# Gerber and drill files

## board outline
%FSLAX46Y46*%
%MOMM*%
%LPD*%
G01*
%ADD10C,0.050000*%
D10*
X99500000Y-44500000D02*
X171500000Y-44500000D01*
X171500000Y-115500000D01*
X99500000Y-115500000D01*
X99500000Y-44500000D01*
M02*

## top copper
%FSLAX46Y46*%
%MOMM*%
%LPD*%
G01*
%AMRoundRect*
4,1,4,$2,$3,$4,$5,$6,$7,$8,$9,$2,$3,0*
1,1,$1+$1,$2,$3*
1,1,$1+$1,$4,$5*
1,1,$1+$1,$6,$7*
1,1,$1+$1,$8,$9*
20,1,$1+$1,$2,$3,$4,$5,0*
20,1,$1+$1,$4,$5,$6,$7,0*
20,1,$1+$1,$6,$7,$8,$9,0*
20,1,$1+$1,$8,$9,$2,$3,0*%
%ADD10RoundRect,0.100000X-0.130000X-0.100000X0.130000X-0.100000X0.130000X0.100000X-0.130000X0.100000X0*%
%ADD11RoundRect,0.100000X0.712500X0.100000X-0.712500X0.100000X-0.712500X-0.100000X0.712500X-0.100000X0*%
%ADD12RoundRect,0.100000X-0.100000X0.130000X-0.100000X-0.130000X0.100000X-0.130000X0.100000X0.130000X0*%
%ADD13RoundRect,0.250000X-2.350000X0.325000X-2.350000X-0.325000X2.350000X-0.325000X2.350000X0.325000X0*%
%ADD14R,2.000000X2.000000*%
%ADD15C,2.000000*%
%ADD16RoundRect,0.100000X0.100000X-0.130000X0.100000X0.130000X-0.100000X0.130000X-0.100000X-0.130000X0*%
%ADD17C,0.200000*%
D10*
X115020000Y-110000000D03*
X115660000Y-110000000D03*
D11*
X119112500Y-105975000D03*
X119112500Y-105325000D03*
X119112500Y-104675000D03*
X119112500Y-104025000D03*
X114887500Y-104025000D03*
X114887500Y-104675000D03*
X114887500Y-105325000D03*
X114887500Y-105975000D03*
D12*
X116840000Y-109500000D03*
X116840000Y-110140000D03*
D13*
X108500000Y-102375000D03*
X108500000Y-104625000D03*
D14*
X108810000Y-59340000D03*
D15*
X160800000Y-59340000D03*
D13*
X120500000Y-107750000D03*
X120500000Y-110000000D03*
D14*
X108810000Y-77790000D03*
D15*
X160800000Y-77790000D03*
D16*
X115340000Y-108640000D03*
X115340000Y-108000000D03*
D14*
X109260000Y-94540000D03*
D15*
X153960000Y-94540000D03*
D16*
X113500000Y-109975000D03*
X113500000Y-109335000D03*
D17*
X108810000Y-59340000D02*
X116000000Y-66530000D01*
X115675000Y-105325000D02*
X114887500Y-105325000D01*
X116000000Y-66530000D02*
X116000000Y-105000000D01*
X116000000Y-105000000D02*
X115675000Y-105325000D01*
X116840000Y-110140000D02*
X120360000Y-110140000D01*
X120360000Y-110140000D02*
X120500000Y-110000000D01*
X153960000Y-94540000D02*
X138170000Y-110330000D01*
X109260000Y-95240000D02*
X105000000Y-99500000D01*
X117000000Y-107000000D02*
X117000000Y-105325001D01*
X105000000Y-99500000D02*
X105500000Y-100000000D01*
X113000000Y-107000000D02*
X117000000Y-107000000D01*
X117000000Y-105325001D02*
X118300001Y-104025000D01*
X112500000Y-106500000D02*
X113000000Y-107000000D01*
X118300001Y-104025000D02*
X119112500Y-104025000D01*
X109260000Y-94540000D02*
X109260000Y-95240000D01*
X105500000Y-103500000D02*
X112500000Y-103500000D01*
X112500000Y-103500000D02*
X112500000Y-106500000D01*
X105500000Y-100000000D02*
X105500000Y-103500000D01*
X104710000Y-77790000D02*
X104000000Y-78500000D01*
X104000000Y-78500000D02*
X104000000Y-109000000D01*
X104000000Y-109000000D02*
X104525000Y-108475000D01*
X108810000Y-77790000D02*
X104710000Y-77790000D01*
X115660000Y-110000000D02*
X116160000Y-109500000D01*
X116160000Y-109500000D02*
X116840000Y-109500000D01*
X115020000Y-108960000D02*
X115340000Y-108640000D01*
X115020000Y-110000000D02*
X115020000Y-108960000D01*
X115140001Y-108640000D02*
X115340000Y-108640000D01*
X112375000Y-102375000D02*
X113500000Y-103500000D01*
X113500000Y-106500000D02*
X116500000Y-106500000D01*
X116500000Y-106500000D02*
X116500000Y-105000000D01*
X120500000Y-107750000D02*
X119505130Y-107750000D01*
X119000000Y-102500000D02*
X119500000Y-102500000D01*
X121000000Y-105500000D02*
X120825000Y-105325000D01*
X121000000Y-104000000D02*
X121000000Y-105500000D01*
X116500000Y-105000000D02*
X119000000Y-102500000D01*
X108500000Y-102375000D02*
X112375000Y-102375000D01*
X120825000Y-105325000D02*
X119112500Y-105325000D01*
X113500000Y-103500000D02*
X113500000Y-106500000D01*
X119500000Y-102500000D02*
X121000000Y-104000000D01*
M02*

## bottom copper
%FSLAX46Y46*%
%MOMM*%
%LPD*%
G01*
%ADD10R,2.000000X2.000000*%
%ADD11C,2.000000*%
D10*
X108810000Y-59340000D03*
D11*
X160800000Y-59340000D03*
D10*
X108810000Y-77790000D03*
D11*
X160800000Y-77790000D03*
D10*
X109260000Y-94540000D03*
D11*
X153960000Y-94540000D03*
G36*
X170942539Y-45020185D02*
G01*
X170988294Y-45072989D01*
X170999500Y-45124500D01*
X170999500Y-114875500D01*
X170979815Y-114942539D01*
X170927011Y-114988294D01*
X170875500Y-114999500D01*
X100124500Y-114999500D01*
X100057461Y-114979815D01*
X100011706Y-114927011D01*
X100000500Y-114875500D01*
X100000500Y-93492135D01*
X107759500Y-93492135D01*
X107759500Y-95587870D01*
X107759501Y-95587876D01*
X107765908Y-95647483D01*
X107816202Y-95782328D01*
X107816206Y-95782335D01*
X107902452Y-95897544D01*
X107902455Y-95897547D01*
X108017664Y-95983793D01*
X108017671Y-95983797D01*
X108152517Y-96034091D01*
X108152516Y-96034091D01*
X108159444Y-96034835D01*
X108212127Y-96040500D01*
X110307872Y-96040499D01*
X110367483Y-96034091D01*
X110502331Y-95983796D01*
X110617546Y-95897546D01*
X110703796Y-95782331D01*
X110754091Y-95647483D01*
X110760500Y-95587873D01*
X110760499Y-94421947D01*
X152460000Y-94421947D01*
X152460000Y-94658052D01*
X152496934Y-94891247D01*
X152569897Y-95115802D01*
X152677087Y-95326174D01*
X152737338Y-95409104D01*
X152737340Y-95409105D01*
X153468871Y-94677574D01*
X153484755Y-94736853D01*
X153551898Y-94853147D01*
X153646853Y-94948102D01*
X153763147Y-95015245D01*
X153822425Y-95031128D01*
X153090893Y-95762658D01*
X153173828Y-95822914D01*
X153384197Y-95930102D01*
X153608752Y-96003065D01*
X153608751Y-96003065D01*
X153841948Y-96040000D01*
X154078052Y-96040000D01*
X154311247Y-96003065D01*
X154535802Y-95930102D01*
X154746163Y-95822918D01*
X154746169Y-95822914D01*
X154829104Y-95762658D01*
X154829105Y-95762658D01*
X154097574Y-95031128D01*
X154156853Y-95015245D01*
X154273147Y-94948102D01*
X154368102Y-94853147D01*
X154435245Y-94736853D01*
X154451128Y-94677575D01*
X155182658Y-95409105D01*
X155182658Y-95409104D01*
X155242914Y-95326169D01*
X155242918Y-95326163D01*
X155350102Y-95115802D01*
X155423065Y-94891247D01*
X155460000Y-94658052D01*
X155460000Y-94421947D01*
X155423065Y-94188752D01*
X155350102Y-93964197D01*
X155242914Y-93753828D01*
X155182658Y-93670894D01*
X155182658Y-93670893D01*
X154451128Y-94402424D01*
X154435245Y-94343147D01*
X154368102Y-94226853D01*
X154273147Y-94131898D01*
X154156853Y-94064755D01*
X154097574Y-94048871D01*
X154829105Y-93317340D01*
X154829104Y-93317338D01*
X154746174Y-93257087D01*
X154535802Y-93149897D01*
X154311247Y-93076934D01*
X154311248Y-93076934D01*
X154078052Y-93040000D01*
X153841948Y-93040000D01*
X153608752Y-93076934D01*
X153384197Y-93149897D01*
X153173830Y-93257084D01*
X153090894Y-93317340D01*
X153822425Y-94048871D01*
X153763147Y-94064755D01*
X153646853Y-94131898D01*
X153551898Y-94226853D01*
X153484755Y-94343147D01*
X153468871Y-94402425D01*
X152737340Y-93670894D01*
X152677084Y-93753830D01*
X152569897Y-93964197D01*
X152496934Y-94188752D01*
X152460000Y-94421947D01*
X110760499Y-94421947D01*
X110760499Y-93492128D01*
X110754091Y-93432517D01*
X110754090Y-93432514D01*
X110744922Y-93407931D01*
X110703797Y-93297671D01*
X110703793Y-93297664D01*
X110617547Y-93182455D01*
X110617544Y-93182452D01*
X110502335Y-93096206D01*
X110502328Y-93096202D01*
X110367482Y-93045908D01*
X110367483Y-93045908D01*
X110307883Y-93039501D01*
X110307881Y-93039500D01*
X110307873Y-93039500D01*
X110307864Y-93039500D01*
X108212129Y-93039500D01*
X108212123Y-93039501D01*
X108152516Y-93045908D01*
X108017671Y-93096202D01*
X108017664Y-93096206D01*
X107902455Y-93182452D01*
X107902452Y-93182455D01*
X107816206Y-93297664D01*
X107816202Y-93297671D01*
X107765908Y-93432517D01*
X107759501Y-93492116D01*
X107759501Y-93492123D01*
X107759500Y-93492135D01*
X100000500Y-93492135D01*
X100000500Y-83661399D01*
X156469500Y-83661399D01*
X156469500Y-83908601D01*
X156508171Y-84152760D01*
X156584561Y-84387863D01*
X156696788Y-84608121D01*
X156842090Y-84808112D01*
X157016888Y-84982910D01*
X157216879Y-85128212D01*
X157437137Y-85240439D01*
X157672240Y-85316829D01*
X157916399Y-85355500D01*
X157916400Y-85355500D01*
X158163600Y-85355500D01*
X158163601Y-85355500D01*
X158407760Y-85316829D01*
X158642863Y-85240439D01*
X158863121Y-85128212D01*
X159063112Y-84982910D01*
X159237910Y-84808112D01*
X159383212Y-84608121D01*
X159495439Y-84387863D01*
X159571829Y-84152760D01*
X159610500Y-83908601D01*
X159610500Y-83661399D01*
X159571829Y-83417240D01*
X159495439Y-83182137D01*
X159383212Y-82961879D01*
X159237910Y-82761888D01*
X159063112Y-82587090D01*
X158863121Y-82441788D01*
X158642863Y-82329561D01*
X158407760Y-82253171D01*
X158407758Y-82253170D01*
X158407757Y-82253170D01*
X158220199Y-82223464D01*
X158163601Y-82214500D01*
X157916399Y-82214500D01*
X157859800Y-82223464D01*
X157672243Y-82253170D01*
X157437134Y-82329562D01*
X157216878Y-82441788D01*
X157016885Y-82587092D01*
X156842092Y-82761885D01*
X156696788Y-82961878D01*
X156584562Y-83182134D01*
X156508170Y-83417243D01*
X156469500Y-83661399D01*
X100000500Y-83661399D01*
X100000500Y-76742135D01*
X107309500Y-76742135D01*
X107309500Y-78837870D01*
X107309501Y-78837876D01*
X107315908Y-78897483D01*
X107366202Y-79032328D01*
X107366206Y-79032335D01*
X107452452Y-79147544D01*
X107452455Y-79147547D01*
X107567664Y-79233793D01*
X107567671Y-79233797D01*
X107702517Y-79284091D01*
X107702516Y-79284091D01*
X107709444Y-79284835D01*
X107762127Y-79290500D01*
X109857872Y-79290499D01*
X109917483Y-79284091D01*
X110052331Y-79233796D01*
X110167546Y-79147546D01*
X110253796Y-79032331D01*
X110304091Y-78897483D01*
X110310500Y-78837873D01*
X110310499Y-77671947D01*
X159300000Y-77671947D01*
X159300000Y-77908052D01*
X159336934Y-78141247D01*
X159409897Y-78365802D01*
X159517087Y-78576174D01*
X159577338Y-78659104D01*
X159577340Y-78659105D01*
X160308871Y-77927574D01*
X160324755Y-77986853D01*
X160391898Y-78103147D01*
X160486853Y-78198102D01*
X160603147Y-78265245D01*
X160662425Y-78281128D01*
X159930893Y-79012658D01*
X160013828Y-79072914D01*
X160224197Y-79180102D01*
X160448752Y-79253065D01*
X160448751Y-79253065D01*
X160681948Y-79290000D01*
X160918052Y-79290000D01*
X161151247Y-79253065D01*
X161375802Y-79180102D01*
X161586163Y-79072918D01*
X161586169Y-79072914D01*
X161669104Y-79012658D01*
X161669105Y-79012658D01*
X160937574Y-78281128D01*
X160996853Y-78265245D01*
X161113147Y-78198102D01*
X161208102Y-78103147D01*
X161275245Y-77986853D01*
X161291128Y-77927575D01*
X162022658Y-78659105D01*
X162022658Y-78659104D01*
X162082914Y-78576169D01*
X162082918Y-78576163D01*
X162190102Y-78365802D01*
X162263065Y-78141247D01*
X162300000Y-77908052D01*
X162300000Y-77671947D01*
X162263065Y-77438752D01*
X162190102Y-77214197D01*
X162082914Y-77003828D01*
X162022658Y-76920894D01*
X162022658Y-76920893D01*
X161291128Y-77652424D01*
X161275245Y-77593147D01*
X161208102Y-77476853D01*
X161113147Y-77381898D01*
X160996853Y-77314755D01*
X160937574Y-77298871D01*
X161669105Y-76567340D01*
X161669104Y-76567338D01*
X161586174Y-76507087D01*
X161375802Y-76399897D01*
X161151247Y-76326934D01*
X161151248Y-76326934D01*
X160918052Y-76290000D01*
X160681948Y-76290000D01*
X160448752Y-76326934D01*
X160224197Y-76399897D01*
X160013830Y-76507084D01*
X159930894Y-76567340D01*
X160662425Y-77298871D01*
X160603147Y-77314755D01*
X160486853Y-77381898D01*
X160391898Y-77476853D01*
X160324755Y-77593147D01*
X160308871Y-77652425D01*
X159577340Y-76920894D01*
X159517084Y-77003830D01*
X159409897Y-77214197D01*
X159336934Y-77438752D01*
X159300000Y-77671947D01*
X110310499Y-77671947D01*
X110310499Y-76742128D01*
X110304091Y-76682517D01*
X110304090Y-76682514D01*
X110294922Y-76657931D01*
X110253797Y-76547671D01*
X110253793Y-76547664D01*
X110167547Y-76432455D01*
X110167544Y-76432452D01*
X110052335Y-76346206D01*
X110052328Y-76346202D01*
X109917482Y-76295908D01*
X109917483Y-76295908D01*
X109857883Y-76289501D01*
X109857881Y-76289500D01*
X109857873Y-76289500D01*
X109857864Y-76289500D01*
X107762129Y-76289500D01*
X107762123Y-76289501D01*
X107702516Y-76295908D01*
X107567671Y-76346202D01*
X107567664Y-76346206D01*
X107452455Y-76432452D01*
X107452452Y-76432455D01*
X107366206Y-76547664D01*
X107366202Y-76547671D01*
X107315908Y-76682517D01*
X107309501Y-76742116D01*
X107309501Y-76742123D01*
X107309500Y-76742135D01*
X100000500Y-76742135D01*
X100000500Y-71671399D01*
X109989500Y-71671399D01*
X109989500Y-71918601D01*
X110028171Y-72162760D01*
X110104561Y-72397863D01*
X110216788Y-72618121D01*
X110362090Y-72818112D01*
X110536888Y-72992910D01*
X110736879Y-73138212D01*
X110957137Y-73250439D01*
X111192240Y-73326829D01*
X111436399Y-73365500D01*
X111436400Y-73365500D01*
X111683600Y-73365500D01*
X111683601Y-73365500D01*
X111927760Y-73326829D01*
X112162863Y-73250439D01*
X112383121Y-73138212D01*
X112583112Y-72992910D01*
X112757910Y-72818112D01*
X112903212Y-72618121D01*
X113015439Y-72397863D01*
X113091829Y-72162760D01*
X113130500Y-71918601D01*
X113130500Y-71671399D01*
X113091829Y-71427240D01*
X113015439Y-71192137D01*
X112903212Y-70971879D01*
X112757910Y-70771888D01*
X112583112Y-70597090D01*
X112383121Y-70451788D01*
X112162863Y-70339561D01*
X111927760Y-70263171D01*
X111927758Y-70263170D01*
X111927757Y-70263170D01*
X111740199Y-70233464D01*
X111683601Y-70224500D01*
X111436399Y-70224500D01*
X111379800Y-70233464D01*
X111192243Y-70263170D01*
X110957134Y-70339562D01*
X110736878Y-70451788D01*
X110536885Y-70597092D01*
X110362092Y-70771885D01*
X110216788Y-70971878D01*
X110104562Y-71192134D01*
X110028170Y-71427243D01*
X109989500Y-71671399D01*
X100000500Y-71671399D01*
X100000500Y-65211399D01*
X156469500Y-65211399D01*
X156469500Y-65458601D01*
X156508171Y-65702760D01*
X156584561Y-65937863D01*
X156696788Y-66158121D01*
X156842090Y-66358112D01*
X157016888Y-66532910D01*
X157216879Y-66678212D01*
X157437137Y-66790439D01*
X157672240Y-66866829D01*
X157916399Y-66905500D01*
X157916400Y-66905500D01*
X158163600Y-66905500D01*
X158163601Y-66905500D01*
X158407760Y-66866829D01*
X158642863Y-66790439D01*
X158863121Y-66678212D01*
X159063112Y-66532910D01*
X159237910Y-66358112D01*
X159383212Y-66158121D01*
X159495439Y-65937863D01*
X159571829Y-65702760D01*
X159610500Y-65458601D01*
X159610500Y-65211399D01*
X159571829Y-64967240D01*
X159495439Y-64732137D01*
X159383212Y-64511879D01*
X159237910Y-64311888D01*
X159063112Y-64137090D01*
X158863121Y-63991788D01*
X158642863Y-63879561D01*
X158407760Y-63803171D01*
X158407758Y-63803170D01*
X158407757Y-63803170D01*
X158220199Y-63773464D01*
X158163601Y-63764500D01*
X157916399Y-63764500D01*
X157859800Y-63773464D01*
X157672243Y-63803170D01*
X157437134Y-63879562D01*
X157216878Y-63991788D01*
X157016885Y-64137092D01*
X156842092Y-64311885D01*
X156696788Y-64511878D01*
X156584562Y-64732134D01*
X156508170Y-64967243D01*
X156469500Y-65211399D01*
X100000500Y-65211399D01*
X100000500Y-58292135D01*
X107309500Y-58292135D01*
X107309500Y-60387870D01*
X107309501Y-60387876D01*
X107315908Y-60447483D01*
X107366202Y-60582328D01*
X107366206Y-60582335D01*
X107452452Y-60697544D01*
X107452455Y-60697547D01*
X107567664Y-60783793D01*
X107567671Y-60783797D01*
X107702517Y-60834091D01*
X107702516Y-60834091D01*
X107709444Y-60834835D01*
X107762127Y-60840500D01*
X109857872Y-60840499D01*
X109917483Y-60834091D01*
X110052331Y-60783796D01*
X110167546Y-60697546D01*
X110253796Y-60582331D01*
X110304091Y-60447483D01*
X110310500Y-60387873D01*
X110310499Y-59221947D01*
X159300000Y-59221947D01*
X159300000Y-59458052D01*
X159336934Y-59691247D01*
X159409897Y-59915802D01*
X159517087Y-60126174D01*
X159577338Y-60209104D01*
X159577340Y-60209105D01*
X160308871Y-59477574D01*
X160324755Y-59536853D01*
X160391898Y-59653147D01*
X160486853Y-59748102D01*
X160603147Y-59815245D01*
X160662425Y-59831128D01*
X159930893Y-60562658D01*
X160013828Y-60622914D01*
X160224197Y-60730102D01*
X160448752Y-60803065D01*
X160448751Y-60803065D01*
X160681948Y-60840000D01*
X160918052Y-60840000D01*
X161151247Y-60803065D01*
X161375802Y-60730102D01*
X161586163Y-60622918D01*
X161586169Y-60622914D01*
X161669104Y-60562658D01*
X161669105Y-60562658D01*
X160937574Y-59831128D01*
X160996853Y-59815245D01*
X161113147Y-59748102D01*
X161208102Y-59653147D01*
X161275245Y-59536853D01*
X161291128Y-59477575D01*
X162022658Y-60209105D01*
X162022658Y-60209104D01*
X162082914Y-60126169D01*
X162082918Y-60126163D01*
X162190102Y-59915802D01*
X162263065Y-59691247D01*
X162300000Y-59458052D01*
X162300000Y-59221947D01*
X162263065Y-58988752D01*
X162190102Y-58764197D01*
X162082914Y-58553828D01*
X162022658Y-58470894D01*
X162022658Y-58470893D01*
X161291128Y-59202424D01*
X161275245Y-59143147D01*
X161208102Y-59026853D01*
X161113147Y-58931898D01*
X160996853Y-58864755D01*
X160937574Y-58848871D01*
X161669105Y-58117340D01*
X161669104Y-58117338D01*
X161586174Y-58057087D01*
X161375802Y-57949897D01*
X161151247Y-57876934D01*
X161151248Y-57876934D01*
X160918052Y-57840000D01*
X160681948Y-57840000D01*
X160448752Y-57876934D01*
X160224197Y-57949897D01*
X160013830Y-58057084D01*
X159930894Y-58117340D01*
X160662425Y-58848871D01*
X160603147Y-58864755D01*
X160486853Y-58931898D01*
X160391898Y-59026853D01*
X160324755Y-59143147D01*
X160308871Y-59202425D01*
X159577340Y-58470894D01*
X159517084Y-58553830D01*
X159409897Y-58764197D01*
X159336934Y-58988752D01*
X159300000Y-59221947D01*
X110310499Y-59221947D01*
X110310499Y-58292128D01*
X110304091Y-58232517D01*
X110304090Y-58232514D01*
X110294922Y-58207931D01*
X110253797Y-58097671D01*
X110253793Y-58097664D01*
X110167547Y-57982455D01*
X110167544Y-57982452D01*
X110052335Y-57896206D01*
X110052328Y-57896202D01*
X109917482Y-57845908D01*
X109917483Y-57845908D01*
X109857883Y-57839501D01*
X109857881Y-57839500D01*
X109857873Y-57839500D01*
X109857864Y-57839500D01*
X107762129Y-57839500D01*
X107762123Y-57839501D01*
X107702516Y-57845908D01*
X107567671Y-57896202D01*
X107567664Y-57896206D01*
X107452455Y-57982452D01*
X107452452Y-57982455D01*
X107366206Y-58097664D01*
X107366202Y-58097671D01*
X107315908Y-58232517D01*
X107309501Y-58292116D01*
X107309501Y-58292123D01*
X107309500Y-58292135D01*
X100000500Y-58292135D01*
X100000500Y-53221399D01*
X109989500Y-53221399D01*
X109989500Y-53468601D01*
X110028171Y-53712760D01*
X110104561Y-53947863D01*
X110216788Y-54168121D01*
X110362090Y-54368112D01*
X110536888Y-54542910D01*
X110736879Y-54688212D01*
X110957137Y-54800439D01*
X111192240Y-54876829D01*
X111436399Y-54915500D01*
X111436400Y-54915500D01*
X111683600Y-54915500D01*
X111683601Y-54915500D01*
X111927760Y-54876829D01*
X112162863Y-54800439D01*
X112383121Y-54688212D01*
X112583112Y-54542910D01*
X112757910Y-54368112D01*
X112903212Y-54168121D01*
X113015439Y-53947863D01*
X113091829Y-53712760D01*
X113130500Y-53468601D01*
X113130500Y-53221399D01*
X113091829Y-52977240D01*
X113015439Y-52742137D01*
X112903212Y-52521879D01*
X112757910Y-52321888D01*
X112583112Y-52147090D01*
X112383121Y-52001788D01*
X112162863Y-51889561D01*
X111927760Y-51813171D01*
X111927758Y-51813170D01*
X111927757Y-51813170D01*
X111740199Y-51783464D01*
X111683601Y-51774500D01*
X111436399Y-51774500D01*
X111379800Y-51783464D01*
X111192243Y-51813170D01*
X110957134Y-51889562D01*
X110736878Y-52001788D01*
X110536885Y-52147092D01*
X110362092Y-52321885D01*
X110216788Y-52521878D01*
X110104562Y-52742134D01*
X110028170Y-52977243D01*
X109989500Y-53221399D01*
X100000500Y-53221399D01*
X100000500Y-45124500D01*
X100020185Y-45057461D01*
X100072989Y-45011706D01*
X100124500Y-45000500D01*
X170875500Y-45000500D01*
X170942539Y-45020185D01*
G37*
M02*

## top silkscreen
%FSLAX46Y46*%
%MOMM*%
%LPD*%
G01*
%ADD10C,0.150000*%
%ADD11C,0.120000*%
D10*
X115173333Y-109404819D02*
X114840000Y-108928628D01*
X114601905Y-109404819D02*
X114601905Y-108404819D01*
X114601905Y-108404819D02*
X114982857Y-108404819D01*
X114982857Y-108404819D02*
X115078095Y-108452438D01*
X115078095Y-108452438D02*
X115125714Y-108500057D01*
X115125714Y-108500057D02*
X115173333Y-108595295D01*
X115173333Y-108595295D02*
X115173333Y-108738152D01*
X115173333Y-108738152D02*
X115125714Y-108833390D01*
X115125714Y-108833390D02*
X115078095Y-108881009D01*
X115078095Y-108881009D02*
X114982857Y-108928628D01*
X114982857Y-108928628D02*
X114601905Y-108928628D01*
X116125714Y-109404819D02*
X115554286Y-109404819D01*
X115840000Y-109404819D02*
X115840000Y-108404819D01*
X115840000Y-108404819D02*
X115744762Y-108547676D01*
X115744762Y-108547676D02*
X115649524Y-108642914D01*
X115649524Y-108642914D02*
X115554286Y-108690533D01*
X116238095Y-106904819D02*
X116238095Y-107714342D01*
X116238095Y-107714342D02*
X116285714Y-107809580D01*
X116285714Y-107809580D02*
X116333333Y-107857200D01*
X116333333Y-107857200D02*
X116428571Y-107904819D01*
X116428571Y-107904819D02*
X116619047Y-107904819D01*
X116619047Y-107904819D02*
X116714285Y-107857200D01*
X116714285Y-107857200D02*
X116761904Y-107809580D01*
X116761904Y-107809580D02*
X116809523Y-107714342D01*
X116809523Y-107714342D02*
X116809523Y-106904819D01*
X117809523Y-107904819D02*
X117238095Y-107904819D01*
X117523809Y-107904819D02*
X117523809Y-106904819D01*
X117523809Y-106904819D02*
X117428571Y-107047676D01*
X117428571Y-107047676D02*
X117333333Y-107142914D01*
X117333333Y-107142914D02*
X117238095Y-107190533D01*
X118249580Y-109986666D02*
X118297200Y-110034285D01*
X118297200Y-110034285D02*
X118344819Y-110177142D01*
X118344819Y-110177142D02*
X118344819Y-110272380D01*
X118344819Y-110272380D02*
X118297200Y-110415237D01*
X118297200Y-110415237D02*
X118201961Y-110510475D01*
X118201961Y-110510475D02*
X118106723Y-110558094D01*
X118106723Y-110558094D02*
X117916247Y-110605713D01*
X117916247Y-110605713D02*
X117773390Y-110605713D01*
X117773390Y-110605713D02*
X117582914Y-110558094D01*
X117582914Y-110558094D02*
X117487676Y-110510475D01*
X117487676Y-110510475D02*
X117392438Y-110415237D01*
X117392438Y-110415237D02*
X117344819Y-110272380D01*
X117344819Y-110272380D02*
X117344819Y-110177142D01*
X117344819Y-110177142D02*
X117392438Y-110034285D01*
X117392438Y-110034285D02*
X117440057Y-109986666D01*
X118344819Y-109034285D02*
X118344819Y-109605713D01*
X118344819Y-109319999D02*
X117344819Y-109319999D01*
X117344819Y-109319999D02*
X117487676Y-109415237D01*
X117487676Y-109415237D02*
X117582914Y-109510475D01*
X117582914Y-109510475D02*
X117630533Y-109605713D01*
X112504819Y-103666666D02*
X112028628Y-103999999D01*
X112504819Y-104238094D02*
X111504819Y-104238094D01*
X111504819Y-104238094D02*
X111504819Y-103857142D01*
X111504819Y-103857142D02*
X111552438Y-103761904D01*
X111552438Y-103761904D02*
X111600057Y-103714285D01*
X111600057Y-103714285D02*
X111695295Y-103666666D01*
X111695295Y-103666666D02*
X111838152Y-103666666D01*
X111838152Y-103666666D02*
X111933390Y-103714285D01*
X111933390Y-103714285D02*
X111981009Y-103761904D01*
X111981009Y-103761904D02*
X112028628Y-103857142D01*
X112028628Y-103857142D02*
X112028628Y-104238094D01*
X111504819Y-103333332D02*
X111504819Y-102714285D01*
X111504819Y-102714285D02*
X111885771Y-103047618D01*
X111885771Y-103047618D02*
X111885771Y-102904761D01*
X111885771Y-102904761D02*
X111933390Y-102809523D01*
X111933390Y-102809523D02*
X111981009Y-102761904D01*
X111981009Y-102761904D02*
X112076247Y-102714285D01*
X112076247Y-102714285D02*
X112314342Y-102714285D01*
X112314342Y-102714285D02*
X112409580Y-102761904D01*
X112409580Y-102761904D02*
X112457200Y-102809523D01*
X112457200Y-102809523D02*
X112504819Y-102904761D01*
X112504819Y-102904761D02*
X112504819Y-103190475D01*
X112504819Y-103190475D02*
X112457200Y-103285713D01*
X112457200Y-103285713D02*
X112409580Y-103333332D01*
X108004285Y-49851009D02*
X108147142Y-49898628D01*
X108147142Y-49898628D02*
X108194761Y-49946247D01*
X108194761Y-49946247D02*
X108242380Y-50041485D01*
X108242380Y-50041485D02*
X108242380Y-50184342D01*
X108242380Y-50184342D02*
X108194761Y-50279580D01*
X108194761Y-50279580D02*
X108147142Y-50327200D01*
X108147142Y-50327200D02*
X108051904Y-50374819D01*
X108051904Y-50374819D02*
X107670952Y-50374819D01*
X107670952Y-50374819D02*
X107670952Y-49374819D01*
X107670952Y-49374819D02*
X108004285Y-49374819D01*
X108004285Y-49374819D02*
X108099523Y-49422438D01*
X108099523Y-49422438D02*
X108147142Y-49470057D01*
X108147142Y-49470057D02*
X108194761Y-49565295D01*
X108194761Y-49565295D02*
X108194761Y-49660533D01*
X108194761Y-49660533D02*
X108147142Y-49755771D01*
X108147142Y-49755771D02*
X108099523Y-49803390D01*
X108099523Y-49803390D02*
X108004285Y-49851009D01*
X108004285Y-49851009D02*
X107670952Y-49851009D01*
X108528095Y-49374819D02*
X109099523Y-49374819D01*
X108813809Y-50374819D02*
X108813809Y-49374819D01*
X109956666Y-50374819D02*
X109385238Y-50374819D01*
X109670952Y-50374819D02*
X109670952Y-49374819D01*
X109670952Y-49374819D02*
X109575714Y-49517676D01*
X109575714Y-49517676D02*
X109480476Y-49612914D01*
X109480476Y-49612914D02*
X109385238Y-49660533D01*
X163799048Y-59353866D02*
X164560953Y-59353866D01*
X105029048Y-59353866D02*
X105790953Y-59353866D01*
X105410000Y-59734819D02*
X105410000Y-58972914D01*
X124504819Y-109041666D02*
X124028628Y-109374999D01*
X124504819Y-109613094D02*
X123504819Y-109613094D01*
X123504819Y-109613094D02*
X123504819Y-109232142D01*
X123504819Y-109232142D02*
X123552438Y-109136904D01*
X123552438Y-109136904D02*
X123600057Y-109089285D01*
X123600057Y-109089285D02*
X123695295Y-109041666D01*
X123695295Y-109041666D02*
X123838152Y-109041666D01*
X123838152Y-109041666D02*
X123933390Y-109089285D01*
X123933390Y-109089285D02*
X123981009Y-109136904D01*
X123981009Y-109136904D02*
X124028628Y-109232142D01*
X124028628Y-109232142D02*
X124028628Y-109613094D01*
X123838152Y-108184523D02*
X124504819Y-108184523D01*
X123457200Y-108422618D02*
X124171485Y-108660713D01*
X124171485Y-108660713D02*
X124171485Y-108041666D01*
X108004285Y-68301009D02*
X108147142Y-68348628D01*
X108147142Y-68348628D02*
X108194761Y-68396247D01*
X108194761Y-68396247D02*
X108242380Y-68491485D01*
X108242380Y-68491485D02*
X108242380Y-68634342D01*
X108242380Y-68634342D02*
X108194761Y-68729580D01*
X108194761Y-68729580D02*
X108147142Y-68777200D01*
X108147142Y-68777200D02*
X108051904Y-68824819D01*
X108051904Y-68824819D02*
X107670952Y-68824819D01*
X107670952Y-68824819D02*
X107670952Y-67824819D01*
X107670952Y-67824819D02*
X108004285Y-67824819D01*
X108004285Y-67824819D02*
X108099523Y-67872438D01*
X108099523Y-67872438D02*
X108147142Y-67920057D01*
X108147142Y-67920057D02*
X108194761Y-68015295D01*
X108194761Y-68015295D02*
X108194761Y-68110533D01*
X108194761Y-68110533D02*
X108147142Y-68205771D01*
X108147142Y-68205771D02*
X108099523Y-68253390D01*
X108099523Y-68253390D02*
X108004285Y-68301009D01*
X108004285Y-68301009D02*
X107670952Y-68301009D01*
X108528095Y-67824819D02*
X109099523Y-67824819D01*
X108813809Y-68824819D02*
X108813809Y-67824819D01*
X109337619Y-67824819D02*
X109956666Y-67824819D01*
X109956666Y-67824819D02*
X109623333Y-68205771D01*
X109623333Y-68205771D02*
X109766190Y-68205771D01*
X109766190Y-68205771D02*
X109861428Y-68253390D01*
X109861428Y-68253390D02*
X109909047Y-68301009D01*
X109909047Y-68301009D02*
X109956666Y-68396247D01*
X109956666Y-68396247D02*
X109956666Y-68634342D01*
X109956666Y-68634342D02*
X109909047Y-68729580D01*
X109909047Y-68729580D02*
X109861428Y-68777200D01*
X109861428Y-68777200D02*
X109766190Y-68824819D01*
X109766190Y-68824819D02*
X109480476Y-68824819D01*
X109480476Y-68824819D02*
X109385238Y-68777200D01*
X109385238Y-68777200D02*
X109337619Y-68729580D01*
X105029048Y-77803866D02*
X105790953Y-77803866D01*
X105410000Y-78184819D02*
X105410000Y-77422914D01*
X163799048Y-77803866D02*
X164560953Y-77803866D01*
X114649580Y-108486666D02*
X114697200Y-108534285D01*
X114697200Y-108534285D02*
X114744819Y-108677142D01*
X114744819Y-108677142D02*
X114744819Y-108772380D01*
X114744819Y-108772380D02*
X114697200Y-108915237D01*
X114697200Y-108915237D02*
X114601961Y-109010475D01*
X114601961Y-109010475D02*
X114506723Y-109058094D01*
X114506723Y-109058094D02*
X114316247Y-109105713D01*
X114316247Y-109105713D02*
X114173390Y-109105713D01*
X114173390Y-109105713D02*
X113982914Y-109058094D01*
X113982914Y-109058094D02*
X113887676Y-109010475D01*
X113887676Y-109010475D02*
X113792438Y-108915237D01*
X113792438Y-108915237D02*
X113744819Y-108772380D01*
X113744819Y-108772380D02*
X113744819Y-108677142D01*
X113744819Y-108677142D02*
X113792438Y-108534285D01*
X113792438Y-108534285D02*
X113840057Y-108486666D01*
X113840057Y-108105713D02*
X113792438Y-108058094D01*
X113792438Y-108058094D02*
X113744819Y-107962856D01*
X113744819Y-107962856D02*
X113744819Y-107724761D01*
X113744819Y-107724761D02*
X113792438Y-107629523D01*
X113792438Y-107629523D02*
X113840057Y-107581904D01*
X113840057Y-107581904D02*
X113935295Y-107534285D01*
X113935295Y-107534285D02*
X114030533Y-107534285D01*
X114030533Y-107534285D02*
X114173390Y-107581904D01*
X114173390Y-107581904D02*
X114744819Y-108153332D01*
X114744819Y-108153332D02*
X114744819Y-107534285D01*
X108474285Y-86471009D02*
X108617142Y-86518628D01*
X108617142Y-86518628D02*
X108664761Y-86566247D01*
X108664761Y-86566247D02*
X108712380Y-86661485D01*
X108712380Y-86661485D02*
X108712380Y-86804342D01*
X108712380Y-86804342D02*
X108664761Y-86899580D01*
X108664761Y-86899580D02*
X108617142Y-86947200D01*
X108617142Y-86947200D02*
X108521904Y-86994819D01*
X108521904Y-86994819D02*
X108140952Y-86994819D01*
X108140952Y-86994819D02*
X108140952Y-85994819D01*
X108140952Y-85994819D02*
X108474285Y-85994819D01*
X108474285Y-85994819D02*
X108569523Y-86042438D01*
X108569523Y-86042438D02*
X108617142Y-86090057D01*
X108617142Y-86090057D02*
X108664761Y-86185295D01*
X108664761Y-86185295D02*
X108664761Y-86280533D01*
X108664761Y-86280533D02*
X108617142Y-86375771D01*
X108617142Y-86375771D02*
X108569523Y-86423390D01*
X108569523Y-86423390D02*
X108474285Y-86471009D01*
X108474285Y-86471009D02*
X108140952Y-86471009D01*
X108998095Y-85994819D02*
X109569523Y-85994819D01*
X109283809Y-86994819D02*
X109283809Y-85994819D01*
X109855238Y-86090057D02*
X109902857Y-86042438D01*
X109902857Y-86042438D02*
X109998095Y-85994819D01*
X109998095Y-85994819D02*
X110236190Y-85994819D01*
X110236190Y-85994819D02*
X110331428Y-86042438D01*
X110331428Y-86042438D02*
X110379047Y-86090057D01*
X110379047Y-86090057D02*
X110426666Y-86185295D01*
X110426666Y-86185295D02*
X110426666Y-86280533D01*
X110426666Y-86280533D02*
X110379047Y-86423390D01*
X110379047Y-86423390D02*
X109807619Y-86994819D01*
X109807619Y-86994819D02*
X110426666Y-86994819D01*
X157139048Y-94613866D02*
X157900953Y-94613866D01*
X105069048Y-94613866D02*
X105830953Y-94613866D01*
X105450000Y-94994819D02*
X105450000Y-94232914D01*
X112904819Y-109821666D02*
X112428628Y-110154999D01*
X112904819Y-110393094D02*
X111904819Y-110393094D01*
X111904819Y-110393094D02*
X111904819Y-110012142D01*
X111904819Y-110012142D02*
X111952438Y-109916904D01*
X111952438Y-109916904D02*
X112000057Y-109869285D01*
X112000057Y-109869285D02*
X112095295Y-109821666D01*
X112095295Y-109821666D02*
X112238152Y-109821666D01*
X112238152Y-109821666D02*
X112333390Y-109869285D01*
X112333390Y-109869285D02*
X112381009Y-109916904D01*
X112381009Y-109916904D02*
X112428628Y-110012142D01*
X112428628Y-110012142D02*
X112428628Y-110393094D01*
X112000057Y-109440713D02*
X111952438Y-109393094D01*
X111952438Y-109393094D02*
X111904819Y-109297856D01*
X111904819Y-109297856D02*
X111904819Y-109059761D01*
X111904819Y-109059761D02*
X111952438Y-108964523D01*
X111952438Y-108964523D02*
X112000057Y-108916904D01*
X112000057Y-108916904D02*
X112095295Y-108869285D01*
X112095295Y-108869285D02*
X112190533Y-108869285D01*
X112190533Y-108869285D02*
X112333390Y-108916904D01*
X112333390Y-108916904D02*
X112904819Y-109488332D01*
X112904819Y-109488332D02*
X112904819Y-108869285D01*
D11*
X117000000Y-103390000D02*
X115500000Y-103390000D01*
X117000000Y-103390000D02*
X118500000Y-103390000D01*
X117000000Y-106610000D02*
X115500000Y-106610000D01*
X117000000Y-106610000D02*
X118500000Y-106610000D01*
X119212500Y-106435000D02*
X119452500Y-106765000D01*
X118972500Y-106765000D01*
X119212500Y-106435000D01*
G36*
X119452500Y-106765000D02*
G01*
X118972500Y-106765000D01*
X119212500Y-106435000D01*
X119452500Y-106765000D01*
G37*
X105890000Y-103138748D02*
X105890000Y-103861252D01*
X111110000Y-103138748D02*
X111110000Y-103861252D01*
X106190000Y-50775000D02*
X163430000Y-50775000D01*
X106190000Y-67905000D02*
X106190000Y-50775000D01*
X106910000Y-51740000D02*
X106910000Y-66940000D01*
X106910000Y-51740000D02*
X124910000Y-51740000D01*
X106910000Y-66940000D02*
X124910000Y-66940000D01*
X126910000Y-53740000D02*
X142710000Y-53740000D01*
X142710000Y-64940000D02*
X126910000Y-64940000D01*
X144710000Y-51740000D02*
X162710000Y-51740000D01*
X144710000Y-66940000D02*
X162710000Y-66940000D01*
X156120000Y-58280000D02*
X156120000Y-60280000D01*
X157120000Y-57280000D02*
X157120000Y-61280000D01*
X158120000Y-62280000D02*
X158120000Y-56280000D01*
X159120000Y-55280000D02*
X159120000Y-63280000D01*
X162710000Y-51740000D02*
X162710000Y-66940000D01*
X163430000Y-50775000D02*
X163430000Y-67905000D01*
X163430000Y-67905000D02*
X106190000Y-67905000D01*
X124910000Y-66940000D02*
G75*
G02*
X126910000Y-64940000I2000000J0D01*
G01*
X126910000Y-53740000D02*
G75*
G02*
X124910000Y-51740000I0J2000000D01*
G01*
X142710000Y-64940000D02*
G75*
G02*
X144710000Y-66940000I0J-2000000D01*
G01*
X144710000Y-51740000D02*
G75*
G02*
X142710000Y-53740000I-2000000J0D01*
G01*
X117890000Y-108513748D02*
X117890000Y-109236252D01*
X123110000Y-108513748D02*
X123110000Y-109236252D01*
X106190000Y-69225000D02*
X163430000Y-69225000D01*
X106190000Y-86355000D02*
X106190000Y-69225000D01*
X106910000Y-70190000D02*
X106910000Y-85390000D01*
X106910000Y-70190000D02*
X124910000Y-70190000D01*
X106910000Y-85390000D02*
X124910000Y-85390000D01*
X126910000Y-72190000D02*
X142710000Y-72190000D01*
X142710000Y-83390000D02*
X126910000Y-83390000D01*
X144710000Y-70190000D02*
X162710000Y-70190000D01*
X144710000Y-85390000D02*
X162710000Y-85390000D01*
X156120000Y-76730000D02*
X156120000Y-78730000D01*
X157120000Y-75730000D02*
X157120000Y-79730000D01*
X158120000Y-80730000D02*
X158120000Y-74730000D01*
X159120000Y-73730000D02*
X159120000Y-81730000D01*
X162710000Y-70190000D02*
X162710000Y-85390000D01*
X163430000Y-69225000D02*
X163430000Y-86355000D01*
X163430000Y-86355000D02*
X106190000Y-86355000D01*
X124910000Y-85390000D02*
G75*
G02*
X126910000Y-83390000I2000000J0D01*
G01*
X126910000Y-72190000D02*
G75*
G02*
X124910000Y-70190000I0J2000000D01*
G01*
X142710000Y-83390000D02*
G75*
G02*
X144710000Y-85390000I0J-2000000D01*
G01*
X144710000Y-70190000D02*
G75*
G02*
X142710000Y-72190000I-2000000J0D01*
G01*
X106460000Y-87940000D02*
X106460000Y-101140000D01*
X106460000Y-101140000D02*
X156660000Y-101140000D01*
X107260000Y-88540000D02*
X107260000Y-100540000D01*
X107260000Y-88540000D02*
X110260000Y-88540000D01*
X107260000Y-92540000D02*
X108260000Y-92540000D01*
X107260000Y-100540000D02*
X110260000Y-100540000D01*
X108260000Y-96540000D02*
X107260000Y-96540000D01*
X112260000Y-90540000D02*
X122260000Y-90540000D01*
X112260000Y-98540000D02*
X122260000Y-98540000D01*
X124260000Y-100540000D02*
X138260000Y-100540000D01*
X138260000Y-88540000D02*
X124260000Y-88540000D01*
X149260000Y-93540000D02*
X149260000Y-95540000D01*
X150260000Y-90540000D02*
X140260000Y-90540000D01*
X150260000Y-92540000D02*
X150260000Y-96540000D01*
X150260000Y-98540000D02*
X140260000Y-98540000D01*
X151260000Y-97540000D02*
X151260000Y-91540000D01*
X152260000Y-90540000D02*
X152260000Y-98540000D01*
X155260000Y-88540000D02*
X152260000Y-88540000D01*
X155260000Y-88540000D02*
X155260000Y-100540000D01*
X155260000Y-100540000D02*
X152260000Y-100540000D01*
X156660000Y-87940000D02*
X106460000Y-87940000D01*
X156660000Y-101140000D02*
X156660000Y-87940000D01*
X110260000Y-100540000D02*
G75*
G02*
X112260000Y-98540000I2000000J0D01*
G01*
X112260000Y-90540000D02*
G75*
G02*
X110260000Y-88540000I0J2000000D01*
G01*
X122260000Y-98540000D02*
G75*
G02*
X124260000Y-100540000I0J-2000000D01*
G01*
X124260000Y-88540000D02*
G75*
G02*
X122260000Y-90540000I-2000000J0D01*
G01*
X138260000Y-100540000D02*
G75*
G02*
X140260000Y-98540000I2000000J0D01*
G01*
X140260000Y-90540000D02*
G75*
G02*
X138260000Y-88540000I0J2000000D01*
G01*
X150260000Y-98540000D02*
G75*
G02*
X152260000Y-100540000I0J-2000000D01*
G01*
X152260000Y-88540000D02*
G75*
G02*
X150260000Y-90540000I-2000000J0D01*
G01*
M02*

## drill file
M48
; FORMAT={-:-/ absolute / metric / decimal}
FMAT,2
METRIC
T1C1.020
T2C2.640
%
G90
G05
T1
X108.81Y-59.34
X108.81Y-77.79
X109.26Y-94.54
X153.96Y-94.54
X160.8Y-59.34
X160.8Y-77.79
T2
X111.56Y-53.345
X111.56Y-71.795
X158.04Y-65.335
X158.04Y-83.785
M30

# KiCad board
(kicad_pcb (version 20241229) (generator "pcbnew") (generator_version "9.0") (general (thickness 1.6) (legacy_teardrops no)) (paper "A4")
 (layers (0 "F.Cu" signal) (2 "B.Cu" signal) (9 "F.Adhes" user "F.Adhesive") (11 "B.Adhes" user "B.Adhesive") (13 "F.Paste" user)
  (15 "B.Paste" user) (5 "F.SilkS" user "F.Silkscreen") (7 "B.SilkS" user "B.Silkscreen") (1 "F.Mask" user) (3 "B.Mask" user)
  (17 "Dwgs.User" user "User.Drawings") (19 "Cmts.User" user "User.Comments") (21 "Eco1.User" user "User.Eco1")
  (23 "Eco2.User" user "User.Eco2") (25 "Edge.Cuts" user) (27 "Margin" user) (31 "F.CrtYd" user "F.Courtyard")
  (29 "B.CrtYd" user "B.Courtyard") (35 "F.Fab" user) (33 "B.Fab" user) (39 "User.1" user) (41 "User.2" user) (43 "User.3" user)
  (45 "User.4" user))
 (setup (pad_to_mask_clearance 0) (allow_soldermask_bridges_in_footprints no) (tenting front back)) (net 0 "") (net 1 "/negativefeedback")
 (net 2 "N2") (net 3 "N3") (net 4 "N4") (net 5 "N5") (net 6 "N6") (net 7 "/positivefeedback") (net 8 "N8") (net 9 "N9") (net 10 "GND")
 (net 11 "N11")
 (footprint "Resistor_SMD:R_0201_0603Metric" (layer "F.Cu") (at 115.34 110)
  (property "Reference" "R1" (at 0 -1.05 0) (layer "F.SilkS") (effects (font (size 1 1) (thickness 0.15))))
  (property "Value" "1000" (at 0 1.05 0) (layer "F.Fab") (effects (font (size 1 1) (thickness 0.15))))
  (pad "" smd roundrect (at -0.345 0) (size 0.318 0.36) (layers "F.Paste") (roundrect_rratio 0.25))
  (pad "" smd roundrect (at 0.345 0) (size 0.318 0.36) (layers "F.Paste") (roundrect_rratio 0.25))
  (pad "1" smd roundrect (at -0.32 0) (size 0.46 0.4) (layers "F.Cu" "F.Mask") (roundrect_rratio 0.25) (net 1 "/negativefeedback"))
  (pad "2" smd roundrect (at 0.32 0) (size 0.46 0.4) (layers "F.Cu" "F.Mask") (roundrect_rratio 0.25) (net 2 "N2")))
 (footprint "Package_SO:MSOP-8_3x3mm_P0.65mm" (layer "F.Cu") (at 117 105 180)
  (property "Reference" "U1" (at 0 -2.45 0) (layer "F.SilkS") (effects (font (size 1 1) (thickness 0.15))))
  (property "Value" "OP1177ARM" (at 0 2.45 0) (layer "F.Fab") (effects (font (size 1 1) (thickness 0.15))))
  (fp_line (start 0 1.61) (end 1.5 1.61) (stroke (width 0.12) (type solid)) (layer "F.SilkS"))
  (fp_line (start 0 1.61) (end -1.5 1.61) (stroke (width 0.12) (type solid)) (layer "F.SilkS"))
  (fp_line (start 0 -1.61) (end 1.5 -1.61) (stroke (width 0.12) (type solid)) (layer "F.SilkS"))
  (fp_line (start 0 -1.61) (end -1.5 -1.61) (stroke (width 0.12) (type solid)) (layer "F.SilkS"))
  (fp_poly
   (pts (xy -2.2125 -1.435) (xy -2.4525 -1.765) (xy -1.9725 -1.765)) (stroke (width 0.12) (type solid)) (fill yes) (layer "F.SilkS"))
  (pad "1" smd roundrect (at -2.1125 -0.975 180) (size 1.625 0.4) (layers "F.Cu" "F.Mask" "F.Paste") (roundrect_rratio 0.25) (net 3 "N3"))
  (pad "2" smd roundrect (at -2.1125 -0.325 180) (size 1.625 0.4) (layers "F.Cu" "F.Mask" "F.Paste") (roundrect_rratio 0.25) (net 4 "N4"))
  (pad "3" smd roundrect (at -2.1125 0.325 180) (size 1.625 0.4) (layers "F.Cu" "F.Mask" "F.Paste") (roundrect_rratio 0.25) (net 2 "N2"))
  (pad "4" smd roundrect (at -2.1125 0.975 180) (size 1.625 0.4) (layers "F.Cu" "F.Mask" "F.Paste") (roundrect_rratio 0.25) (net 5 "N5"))
  (pad "5" smd roundrect (at 2.1125 0.975 180) (size 1.625 0.4) (layers "F.Cu" "F.Mask" "F.Paste") (roundrect_rratio 0.25) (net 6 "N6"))
  (pad "6" smd roundrect (at 2.1125 0.325 180) (size 1.625 0.4) (layers "F.Cu" "F.Mask" "F.Paste") (roundrect_rratio 0.25)
   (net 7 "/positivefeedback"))
  (pad "7" smd roundrect (at 2.1125 -0.325 180) (size 1.625 0.4) (layers "F.Cu" "F.Mask" "F.Paste") (roundrect_rratio 0.25) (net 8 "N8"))
  (pad "8" smd roundrect (at 2.1125 -0.975 180) (size 1.625 0.4) (layers "F.Cu" "F.Mask" "F.Paste") (roundrect_rratio 0.25) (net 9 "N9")))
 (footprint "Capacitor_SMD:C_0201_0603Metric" (layer "F.Cu") (at 116.84 109.82 -90)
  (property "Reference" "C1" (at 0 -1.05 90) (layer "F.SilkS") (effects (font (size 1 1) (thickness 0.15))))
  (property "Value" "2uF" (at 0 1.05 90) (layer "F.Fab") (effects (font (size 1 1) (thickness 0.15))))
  (pad "" smd roundrect (at -0.345 0 270) (size 0.318 0.36) (layers "F.Paste") (roundrect_rratio 0.25))
  (pad "" smd roundrect (at 0.345 0 270) (size 0.318 0.36) (layers "F.Paste") (roundrect_rratio 0.25))
  (pad "1" smd roundrect (at -0.32 0 270) (size 0.46 0.4) (layers "F.Cu" "F.Mask") (roundrect_rratio 0.25) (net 2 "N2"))
  (pad "2" smd roundrect (at 0.32 0 270) (size 0.46 0.4) (layers "F.Cu" "F.Mask") (roundrect_rratio 0.25) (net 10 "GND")))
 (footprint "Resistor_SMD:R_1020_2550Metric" (layer "F.Cu") (at 108.5 103.5 -90)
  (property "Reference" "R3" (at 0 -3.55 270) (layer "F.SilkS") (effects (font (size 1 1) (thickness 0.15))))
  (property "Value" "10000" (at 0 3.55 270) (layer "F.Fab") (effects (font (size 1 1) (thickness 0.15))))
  (fp_line (start -0.361252 2.61) (end 0.361252 2.61) (stroke (width 0.12) (type solid)) (layer "F.SilkS"))
  (fp_line (start -0.361252 -2.61) (end 0.361252 -2.61) (stroke (width 0.12) (type solid)) (layer "F.SilkS"))
  (pad "1" smd roundrect (at -1.125 0 270) (size 1.15 5.2) (layers "F.Cu" "F.Mask" "F.Paste") (roundrect_rratio 0.217391) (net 4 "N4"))
  (pad "2" smd roundrect (at 1.125 0 270) (size 1.15 5.2) (layers "F.Cu" "F.Mask" "F.Paste") (roundrect_rratio 0.217391)
   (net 7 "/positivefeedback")))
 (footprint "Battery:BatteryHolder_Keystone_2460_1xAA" (layer "F.Cu") (at 108.81 59.34)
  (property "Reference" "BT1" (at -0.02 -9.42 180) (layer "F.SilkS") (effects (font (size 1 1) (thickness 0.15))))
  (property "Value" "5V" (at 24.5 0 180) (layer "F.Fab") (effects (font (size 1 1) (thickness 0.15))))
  (fp_line (start -2.62 -8.565) (end 54.62 -8.565) (stroke (width 0.12) (type solid)) (layer "F.SilkS"))
  (fp_line (start -2.62 8.565) (end -2.62 -8.565) (stroke (width 0.12) (type solid)) (layer "F.SilkS"))
  (fp_line (start -1.9 -7.6) (end -1.9 7.6) (stroke (width 0.12) (type solid)) (layer "F.SilkS"))
  (fp_line (start -1.9 -7.6) (end 16.1 -7.6) (stroke (width 0.12) (type solid)) (layer "F.SilkS"))
  (fp_line (start -1.9 7.6) (end 16.1 7.6) (stroke (width 0.12) (type solid)) (layer "F.SilkS"))
  (fp_line (start 18.1 -5.6) (end 33.9 -5.6) (stroke (width 0.12) (type solid)) (layer "F.SilkS"))
  (fp_line (start 33.9 5.6) (end 18.1 5.6) (stroke (width 0.12) (type solid)) (layer "F.SilkS"))
  (fp_line (start 35.9 -7.6) (end 53.9 -7.6) (stroke (width 0.12) (type solid)) (layer "F.SilkS"))
  (fp_line (start 35.9 7.6) (end 53.9 7.6) (stroke (width 0.12) (type solid)) (layer "F.SilkS"))
  (fp_line (start 47.31 -1.06) (end 47.31 0.94) (stroke (width 0.12) (type solid)) (layer "F.SilkS"))
  (fp_line (start 48.31 -2.06) (end 48.31 1.94) (stroke (width 0.12) (type solid)) (layer "F.SilkS"))
  (fp_line (start 49.31 2.94) (end 49.31 -3.06) (stroke (width 0.12) (type solid)) (layer "F.SilkS"))
  (fp_line (start 50.31 -4.06) (end 50.31 3.94) (stroke (width 0.12) (type solid)) (layer "F.SilkS"))
  (fp_line (start 53.9 -7.6) (end 53.9 7.6) (stroke (width 0.12) (type solid)) (layer "F.SilkS"))
  (fp_line (start 54.62 -8.565) (end 54.62 8.565) (stroke (width 0.12) (type solid)) (layer "F.SilkS"))
  (fp_line (start 54.62 8.565) (end -2.62 8.565) (stroke (width 0.12) (type solid)) (layer "F.SilkS"))
  (fp_arc (start 16.1 7.6) (mid 16.685786 6.185786) (end 18.1 5.6) (stroke (width 0.12) (type solid)) (layer "F.SilkS"))
  (fp_arc (start 18.1 -5.6) (mid 16.685786 -6.185786) (end 16.1 -7.6) (stroke (width 0.12) (type solid)) (layer "F.SilkS"))
  (fp_arc (start 33.9 5.6) (mid 35.314214 6.185786) (end 35.9 7.6) (stroke (width 0.12) (type solid)) (layer "F.SilkS"))
  (fp_arc (start 35.9 -7.6) (mid 35.314214 -6.185786) (end 33.9 -5.6) (stroke (width 0.12) (type solid)) (layer "F.SilkS"))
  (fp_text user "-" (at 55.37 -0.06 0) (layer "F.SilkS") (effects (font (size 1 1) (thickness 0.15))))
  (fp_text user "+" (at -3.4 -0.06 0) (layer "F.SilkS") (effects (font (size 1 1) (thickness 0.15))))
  (pad "" np_thru_hole circle (at 2.75 -5.995 90) (size 2.64 2.64) (drill 2.64) (layers "*.Cu" "*.Mask"))
  (pad "" np_thru_hole circle (at 49.23 5.995) (size 2.64 2.64) (drill 2.64) (layers "*.Cu" "*.Mask"))
  (pad "1" thru_hole rect (at 0 0 180) (size 2 2) (drill 1.02) (layers "*.Cu" "*.Mask") (remove_unused_layers no) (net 8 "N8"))
  (pad "2" thru_hole circle (at 51.99 0 180) (size 2 2) (drill 1.02) (layers "*.Cu" "*.Mask") (remove_unused_layers no) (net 10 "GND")))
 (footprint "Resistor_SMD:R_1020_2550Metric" (layer "F.Cu") (at 120.5 108.875 -90)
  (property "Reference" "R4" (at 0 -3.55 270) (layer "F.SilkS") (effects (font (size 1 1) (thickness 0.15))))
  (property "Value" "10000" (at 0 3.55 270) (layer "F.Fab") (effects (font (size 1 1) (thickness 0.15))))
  (fp_line (start -0.361252 2.61) (end 0.361252 2.61) (stroke (width 0.12) (type solid)) (layer "F.SilkS"))
  (fp_line (start -0.361252 -2.61) (end 0.361252 -2.61) (stroke (width 0.12) (type solid)) (layer "F.SilkS"))
  (pad "1" smd roundrect (at -1.125 0 270) (size 1.15 5.2) (layers "F.Cu" "F.Mask" "F.Paste") (roundrect_rratio 0.217391) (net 4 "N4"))
  (pad "2" smd roundrect (at 1.125 0 270) (size 1.15 5.2) (layers "F.Cu" "F.Mask" "F.Paste") (roundrect_rratio 0.217391) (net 10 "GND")))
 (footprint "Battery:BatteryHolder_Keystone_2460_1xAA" (layer "F.Cu") (at 108.81 77.79)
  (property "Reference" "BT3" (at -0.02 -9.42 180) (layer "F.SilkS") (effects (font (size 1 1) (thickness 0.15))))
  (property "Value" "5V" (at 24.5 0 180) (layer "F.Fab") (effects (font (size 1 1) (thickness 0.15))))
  (fp_line (start -2.62 -8.565) (end 54.62 -8.565) (stroke (width 0.12) (type solid)) (layer "F.SilkS"))
  (fp_line (start -2.62 8.565) (end -2.62 -8.565) (stroke (width 0.12) (type solid)) (layer "F.SilkS"))
  (fp_line (start -1.9 -7.6) (end -1.9 7.6) (stroke (width 0.12) (type solid)) (layer "F.SilkS"))
  (fp_line (start -1.9 -7.6) (end 16.1 -7.6) (stroke (width 0.12) (type solid)) (layer "F.SilkS"))
  (fp_line (start -1.9 7.6) (end 16.1 7.6) (stroke (width 0.12) (type solid)) (layer "F.SilkS"))
  (fp_line (start 18.1 -5.6) (end 33.9 -5.6) (stroke (width 0.12) (type solid)) (layer "F.SilkS"))
  (fp_line (start 33.9 5.6) (end 18.1 5.6) (stroke (width 0.12) (type solid)) (layer "F.SilkS"))
  (fp_line (start 35.9 -7.6) (end 53.9 -7.6) (stroke (width 0.12) (type solid)) (layer "F.SilkS"))
  (fp_line (start 35.9 7.6) (end 53.9 7.6) (stroke (width 0.12) (type solid)) (layer "F.SilkS"))
  (fp_line (start 47.31 -1.06) (end 47.31 0.94) (stroke (width 0.12) (type solid)) (layer "F.SilkS"))
  (fp_line (start 48.31 -2.06) (end 48.31 1.94) (stroke (width 0.12) (type solid)) (layer "F.SilkS"))
  (fp_line (start 49.31 2.94) (end 49.31 -3.06) (stroke (width 0.12) (type solid)) (layer "F.SilkS"))
  (fp_line (start 50.31 -4.06) (end 50.31 3.94) (stroke (width 0.12) (type solid)) (layer "F.SilkS"))
  (fp_line (start 53.9 -7.6) (end 53.9 7.6) (stroke (width 0.12) (type solid)) (layer "F.SilkS"))
  (fp_line (start 54.62 -8.565) (end 54.62 8.565) (stroke (width 0.12) (type solid)) (layer "F.SilkS"))
  (fp_line (start 54.62 8.565) (end -2.62 8.565) (stroke (width 0.12) (type solid)) (layer "F.SilkS"))
  (fp_arc (start 16.1 7.6) (mid 16.685786 6.185786) (end 18.1 5.6) (stroke (width 0.12) (type solid)) (layer "F.SilkS"))
  (fp_arc (start 18.1 -5.6) (mid 16.685786 -6.185786) (end 16.1 -7.6) (stroke (width 0.12) (type solid)) (layer "F.SilkS"))
  (fp_arc (start 33.9 5.6) (mid 35.314214 6.185786) (end 35.9 7.6) (stroke (width 0.12) (type solid)) (layer "F.SilkS"))
  (fp_arc (start 35.9 -7.6) (mid 35.314214 -6.185786) (end 33.9 -5.6) (stroke (width 0.12) (type solid)) (layer "F.SilkS"))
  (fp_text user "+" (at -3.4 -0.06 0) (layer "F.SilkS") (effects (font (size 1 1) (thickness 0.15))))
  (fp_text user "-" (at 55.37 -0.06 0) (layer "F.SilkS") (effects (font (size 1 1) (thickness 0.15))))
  (pad "" np_thru_hole circle (at 2.75 -5.995 90) (size 2.64 2.64) (drill 2.64) (layers "*.Cu" "*.Mask"))
  (pad "" np_thru_hole circle (at 49.23 5.995) (size 2.64 2.64) (drill 2.64) (layers "*.Cu" "*.Mask"))
  (pad "1" thru_hole rect (at 0 0 180) (size 2 2) (drill 1.02) (layers "*.Cu" "*.Mask") (remove_unused_layers no) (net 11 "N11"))
  (pad "2" thru_hole circle (at 51.99 0 180) (size 2 2) (drill 1.02) (layers "*.Cu" "*.Mask") (remove_unused_layers no) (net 10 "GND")))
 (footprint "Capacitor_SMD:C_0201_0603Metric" (layer "F.Cu") (at 115.34 108.32 90)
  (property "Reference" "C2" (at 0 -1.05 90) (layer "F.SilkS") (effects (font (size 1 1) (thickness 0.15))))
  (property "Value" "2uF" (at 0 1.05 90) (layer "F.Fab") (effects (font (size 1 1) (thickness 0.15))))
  (pad "" smd roundrect (at -0.345 0 90) (size 0.318 0.36) (layers "F.Paste") (roundrect_rratio 0.25))
  (pad "" smd roundrect (at 0.345 0 90) (size 0.318 0.36) (layers "F.Paste") (roundrect_rratio 0.25))
  (pad "1" smd roundrect (at -0.32 0 90) (size 0.46 0.4) (layers "F.Cu" "F.Mask") (roundrect_rratio 0.25) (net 1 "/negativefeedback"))
  (pad "2" smd roundrect (at 0.32 0 90) (size 0.46 0.4) (layers "F.Cu" "F.Mask") (roundrect_rratio 0.25) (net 7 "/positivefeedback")))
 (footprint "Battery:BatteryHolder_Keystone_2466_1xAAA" (layer "F.Cu") (at 109.26 94.54)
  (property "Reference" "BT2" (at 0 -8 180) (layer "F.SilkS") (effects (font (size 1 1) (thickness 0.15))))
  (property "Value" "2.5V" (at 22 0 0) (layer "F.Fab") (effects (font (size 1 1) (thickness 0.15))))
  (fp_line (start -2.8 -6.6) (end -2.8 6.6) (stroke (width 0.12) (type solid)) (layer "F.SilkS"))
  (fp_line (start -2.8 6.6) (end 47.4 6.6) (stroke (width 0.12) (type solid)) (layer "F.SilkS"))
  (fp_line (start -2 -6) (end -2 6) (stroke (width 0.12) (type solid)) (layer "F.SilkS"))
  (fp_line (start -2 -6) (end 1 -6) (stroke (width 0.12) (type solid)) (layer "F.SilkS"))
  (fp_line (start -2 -2) (end -1 -2) (stroke (width 0.12) (type solid)) (layer "F.SilkS"))
  (fp_line (start -2 6) (end 1 6) (stroke (width 0.12) (type solid)) (layer "F.SilkS"))
  (fp_line (start -1 2) (end -2 2) (stroke (width 0.12) (type solid)) (layer "F.SilkS"))
  (fp_line (start 3 -4) (end 13 -4) (stroke (width 0.12) (type solid)) (layer "F.SilkS"))
  (fp_line (start 3 4) (end 13 4) (stroke (width 0.12) (type solid)) (layer "F.SilkS"))
  (fp_line (start 15 6) (end 29 6) (stroke (width 0.12) (type solid)) (layer "F.SilkS"))
  (fp_line (start 29 -6) (end 15 -6) (stroke (width 0.12) (type solid)) (layer "F.SilkS"))
  (fp_line (start 40 -1) (end 40 1) (stroke (width 0.12) (type solid)) (layer "F.SilkS"))
  (fp_line (start 41 -4) (end 31 -4) (stroke (width 0.12) (type solid)) (layer "F.SilkS"))
  (fp_line (start 41 -2) (end 41 2) (stroke (width 0.12) (type solid)) (layer "F.SilkS"))
  (fp_line (start 41 4) (end 31 4) (stroke (width 0.12) (type solid)) (layer "F.SilkS"))
  (fp_line (start 42 3) (end 42 -3) (stroke (width 0.12) (type solid)) (layer "F.SilkS"))
  (fp_line (start 43 -4) (end 43 4) (stroke (width 0.12) (type solid)) (layer "F.SilkS"))
  (fp_line (start 46 -6) (end 43 -6) (stroke (width 0.12) (type solid)) (layer "F.SilkS"))
  (fp_line (start 46 -6) (end 46 6) (stroke (width 0.12) (type solid)) (layer "F.SilkS"))
  (fp_line (start 46 6) (end 43 6) (stroke (width 0.12) (type solid)) (layer "F.SilkS"))
  (fp_line (start 47.4 -6.6) (end -2.8 -6.6) (stroke (width 0.12) (type solid)) (layer "F.SilkS"))
  (fp_line (start 47.4 6.6) (end 47.4 -6.6) (stroke (width 0.12) (type solid)) (layer "F.SilkS"))
  (fp_arc (start 1 6) (mid 1.585786 4.585786) (end 3 4) (stroke (width 0.12) (type solid)) (layer "F.SilkS"))
  (fp_arc (start 3 -4) (mid 1.585786 -4.585786) (end 1 -6) (stroke (width 0.12) (type solid)) (layer "F.SilkS"))
  (fp_arc (start 13 4) (mid 14.414214 4.585786) (end 15 6) (stroke (width 0.12) (type solid)) (layer "F.SilkS"))
  (fp_arc (start 15 -6) (mid 14.414214 -4.585786) (end 13 -4) (stroke (width 0.12) (type solid)) (layer "F.SilkS"))
  (fp_arc (start 29 6) (mid 29.585786 4.585786) (end 31 4) (stroke (width 0.12) (type solid)) (layer "F.SilkS"))
  (fp_arc (start 31 -4) (mid 29.585786 -4.585786) (end 29 -6) (stroke (width 0.12) (type solid)) (layer "F.SilkS"))
  (fp_arc (start 41 4) (mid 42.414214 4.585786) (end 43 6) (stroke (width 0.12) (type solid)) (layer "F.SilkS"))
  (fp_arc (start 43 -6) (mid 42.414214 -4.585786) (end 41 -4) (stroke (width 0.12) (type solid)) (layer "F.SilkS"))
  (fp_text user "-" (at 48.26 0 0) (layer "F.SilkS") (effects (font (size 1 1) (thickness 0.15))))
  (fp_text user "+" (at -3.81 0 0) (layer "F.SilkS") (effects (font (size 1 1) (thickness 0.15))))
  (pad "1" thru_hole rect (at 0 0) (size 2 2) (drill 1.02) (layers "*.Cu" "*.Mask") (remove_unused_layers no) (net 5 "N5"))
  (pad "2" thru_hole circle (at 44.7 0) (size 2 2) (drill 1.02) (layers "*.Cu" "*.Mask") (remove_unused_layers no) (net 10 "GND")))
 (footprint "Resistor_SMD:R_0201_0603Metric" (layer "F.Cu") (at 113.5 109.655 90)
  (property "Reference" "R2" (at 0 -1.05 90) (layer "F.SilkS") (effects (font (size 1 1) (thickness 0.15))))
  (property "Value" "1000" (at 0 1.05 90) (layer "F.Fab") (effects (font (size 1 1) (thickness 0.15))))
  (pad "" smd roundrect (at -0.345 0 90) (size 0.318 0.36) (layers "F.Paste") (roundrect_rratio 0.25))
  (pad "" smd roundrect (at 0.345 0 90) (size 0.318 0.36) (layers "F.Paste") (roundrect_rratio 0.25))
  (pad "1" smd roundrect (at -0.32 0 90) (size 0.46 0.4) (layers "F.Cu" "F.Mask") (roundrect_rratio 0.25) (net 11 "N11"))
  (pad "2" smd roundrect (at 0.32 0 90) (size 0.46 0.4) (layers "F.Cu" "F.Mask") (roundrect_rratio 0.25) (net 1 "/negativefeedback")))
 (gr_rect (start 99.5 44.5) (end 171.5 115.5) (stroke (width 0.05) (type default)) (fill no) (layer "Edge.Cuts"))
 (segment (start 108.81 59.34) (end 116 66.53) (width 0.2) (layer "F.Cu") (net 8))
 (segment (start 115.675 105.325) (end 114.8875 105.325) (width 0.2) (layer "F.Cu") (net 8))
 (segment (start 116 66.53) (end 116 105) (width 0.2) (layer "F.Cu") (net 8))
 (segment (start 116 105) (end 115.675 105.325) (width 0.2) (layer "F.Cu") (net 8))
 (segment (start 116.84 110.14) (end 120.36 110.14) (width 0.2) (layer "F.Cu") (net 10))
 (segment (start 120.36 110.14) (end 120.5 110) (width 0.2) (layer "F.Cu") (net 10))
 (segment (start 153.96 94.54) (end 138.17 110.33) (width 0.2) (layer "F.Cu") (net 10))
 (segment (start 109.26 95.24) (end 105 99.5) (width 0.2) (layer "F.Cu") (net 5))
 (segment (start 117 107) (end 117 105.325001) (width 0.2) (layer "F.Cu") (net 5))
 (segment (start 105 99.5) (end 105.5 100) (width 0.2) (layer "F.Cu") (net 5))
 (segment (start 113 107) (end 117 107) (width 0.2) (layer "F.Cu") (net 5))
 (segment (start 117 105.325001) (end 118.300001 104.025) (width 0.2) (layer "F.Cu") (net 5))
 (segment (start 112.5 106.5) (end 113 107) (width 0.2) (layer "F.Cu") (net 5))
 (segment (start 118.300001 104.025) (end 119.1125 104.025) (width 0.2) (layer "F.Cu") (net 5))
 (segment (start 109.26 94.54) (end 109.26 95.24) (width 0.2) (layer "F.Cu") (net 5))
 (segment (start 105.5 103.5) (end 112.5 103.5) (width 0.2) (layer "F.Cu") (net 5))
 (segment (start 112.5 103.5) (end 112.5 106.5) (width 0.2) (layer "F.Cu") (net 5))
 (segment (start 105.5 100) (end 105.5 103.5) (width 0.2) (layer "F.Cu") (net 5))
 (segment (start 104.71 77.79) (end 104 78.5) (width 0.2) (layer "F.Cu") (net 11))
 (segment (start 104 78.5) (end 104 109) (width 0.2) (layer "F.Cu") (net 11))
 (segment (start 104 109) (end 104.525 108.475) (width 0.2) (layer "F.Cu") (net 11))
 (segment (start 108.81 77.79) (end 104.71 77.79) (width 0.2) (layer "F.Cu") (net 11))
 (segment (start 115.66 110) (end 116.16 109.5) (width 0.2) (layer "F.Cu") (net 2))
 (segment (start 116.16 109.5) (end 116.84 109.5) (width 0.2) (layer "F.Cu") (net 2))
 (segment (start 115.02 108.96) (end 115.34 108.64) (width 0.2) (layer "F.Cu") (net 1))
 (segment (start 115.02 110) (end 115.02 108.96) (width 0.2) (layer "F.Cu") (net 1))
 (segment (start 115.140001 108.64) (end 115.34 108.64) (width 0.2) (layer "F.Cu") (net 1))
 (segment (start 112.375 102.375) (end 113.5 103.5) (width 0.2) (layer "F.Cu") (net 4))
 (segment (start 113.5 106.5) (end 116.5 106.5) (width 0.2) (layer "F.Cu") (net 4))
 (segment (start 116.5 106.5) (end 116.5 105) (width 0.2) (layer "F.Cu") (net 4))
 (segment (start 120.5 107.75) (end 119.50513 107.75) (width 0.2) (layer "F.Cu") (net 4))
 (segment (start 119 102.5) (end 119.5 102.5) (width 0.2) (layer "F.Cu") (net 4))
 (segment (start 121 105.5) (end 120.825 105.325) (width 0.2) (layer "F.Cu") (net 4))
 (segment (start 121 104) (end 121 105.5) (width 0.2) (layer "F.Cu") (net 4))
 (segment (start 116.5 105) (end 119 102.5) (width 0.2) (layer "F.Cu") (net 4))
 (segment (start 108.5 102.375) (end 112.375 102.375) (width 0.2) (layer "F.Cu") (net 4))
 (segment (start 120.825 105.325) (end 119.1125 105.325) (width 0.2) (layer "F.Cu") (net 4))
 (segment (start 113.5 103.5) (end 113.5 106.5) (width 0.2) (layer "F.Cu") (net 4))
 (segment (start 119.5 102.5) (end 121 104) (width 0.2) (layer "F.Cu") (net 4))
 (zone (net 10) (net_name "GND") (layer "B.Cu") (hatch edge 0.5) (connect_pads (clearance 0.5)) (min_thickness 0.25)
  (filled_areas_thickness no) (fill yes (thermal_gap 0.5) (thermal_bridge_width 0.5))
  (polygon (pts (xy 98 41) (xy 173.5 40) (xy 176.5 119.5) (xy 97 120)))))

